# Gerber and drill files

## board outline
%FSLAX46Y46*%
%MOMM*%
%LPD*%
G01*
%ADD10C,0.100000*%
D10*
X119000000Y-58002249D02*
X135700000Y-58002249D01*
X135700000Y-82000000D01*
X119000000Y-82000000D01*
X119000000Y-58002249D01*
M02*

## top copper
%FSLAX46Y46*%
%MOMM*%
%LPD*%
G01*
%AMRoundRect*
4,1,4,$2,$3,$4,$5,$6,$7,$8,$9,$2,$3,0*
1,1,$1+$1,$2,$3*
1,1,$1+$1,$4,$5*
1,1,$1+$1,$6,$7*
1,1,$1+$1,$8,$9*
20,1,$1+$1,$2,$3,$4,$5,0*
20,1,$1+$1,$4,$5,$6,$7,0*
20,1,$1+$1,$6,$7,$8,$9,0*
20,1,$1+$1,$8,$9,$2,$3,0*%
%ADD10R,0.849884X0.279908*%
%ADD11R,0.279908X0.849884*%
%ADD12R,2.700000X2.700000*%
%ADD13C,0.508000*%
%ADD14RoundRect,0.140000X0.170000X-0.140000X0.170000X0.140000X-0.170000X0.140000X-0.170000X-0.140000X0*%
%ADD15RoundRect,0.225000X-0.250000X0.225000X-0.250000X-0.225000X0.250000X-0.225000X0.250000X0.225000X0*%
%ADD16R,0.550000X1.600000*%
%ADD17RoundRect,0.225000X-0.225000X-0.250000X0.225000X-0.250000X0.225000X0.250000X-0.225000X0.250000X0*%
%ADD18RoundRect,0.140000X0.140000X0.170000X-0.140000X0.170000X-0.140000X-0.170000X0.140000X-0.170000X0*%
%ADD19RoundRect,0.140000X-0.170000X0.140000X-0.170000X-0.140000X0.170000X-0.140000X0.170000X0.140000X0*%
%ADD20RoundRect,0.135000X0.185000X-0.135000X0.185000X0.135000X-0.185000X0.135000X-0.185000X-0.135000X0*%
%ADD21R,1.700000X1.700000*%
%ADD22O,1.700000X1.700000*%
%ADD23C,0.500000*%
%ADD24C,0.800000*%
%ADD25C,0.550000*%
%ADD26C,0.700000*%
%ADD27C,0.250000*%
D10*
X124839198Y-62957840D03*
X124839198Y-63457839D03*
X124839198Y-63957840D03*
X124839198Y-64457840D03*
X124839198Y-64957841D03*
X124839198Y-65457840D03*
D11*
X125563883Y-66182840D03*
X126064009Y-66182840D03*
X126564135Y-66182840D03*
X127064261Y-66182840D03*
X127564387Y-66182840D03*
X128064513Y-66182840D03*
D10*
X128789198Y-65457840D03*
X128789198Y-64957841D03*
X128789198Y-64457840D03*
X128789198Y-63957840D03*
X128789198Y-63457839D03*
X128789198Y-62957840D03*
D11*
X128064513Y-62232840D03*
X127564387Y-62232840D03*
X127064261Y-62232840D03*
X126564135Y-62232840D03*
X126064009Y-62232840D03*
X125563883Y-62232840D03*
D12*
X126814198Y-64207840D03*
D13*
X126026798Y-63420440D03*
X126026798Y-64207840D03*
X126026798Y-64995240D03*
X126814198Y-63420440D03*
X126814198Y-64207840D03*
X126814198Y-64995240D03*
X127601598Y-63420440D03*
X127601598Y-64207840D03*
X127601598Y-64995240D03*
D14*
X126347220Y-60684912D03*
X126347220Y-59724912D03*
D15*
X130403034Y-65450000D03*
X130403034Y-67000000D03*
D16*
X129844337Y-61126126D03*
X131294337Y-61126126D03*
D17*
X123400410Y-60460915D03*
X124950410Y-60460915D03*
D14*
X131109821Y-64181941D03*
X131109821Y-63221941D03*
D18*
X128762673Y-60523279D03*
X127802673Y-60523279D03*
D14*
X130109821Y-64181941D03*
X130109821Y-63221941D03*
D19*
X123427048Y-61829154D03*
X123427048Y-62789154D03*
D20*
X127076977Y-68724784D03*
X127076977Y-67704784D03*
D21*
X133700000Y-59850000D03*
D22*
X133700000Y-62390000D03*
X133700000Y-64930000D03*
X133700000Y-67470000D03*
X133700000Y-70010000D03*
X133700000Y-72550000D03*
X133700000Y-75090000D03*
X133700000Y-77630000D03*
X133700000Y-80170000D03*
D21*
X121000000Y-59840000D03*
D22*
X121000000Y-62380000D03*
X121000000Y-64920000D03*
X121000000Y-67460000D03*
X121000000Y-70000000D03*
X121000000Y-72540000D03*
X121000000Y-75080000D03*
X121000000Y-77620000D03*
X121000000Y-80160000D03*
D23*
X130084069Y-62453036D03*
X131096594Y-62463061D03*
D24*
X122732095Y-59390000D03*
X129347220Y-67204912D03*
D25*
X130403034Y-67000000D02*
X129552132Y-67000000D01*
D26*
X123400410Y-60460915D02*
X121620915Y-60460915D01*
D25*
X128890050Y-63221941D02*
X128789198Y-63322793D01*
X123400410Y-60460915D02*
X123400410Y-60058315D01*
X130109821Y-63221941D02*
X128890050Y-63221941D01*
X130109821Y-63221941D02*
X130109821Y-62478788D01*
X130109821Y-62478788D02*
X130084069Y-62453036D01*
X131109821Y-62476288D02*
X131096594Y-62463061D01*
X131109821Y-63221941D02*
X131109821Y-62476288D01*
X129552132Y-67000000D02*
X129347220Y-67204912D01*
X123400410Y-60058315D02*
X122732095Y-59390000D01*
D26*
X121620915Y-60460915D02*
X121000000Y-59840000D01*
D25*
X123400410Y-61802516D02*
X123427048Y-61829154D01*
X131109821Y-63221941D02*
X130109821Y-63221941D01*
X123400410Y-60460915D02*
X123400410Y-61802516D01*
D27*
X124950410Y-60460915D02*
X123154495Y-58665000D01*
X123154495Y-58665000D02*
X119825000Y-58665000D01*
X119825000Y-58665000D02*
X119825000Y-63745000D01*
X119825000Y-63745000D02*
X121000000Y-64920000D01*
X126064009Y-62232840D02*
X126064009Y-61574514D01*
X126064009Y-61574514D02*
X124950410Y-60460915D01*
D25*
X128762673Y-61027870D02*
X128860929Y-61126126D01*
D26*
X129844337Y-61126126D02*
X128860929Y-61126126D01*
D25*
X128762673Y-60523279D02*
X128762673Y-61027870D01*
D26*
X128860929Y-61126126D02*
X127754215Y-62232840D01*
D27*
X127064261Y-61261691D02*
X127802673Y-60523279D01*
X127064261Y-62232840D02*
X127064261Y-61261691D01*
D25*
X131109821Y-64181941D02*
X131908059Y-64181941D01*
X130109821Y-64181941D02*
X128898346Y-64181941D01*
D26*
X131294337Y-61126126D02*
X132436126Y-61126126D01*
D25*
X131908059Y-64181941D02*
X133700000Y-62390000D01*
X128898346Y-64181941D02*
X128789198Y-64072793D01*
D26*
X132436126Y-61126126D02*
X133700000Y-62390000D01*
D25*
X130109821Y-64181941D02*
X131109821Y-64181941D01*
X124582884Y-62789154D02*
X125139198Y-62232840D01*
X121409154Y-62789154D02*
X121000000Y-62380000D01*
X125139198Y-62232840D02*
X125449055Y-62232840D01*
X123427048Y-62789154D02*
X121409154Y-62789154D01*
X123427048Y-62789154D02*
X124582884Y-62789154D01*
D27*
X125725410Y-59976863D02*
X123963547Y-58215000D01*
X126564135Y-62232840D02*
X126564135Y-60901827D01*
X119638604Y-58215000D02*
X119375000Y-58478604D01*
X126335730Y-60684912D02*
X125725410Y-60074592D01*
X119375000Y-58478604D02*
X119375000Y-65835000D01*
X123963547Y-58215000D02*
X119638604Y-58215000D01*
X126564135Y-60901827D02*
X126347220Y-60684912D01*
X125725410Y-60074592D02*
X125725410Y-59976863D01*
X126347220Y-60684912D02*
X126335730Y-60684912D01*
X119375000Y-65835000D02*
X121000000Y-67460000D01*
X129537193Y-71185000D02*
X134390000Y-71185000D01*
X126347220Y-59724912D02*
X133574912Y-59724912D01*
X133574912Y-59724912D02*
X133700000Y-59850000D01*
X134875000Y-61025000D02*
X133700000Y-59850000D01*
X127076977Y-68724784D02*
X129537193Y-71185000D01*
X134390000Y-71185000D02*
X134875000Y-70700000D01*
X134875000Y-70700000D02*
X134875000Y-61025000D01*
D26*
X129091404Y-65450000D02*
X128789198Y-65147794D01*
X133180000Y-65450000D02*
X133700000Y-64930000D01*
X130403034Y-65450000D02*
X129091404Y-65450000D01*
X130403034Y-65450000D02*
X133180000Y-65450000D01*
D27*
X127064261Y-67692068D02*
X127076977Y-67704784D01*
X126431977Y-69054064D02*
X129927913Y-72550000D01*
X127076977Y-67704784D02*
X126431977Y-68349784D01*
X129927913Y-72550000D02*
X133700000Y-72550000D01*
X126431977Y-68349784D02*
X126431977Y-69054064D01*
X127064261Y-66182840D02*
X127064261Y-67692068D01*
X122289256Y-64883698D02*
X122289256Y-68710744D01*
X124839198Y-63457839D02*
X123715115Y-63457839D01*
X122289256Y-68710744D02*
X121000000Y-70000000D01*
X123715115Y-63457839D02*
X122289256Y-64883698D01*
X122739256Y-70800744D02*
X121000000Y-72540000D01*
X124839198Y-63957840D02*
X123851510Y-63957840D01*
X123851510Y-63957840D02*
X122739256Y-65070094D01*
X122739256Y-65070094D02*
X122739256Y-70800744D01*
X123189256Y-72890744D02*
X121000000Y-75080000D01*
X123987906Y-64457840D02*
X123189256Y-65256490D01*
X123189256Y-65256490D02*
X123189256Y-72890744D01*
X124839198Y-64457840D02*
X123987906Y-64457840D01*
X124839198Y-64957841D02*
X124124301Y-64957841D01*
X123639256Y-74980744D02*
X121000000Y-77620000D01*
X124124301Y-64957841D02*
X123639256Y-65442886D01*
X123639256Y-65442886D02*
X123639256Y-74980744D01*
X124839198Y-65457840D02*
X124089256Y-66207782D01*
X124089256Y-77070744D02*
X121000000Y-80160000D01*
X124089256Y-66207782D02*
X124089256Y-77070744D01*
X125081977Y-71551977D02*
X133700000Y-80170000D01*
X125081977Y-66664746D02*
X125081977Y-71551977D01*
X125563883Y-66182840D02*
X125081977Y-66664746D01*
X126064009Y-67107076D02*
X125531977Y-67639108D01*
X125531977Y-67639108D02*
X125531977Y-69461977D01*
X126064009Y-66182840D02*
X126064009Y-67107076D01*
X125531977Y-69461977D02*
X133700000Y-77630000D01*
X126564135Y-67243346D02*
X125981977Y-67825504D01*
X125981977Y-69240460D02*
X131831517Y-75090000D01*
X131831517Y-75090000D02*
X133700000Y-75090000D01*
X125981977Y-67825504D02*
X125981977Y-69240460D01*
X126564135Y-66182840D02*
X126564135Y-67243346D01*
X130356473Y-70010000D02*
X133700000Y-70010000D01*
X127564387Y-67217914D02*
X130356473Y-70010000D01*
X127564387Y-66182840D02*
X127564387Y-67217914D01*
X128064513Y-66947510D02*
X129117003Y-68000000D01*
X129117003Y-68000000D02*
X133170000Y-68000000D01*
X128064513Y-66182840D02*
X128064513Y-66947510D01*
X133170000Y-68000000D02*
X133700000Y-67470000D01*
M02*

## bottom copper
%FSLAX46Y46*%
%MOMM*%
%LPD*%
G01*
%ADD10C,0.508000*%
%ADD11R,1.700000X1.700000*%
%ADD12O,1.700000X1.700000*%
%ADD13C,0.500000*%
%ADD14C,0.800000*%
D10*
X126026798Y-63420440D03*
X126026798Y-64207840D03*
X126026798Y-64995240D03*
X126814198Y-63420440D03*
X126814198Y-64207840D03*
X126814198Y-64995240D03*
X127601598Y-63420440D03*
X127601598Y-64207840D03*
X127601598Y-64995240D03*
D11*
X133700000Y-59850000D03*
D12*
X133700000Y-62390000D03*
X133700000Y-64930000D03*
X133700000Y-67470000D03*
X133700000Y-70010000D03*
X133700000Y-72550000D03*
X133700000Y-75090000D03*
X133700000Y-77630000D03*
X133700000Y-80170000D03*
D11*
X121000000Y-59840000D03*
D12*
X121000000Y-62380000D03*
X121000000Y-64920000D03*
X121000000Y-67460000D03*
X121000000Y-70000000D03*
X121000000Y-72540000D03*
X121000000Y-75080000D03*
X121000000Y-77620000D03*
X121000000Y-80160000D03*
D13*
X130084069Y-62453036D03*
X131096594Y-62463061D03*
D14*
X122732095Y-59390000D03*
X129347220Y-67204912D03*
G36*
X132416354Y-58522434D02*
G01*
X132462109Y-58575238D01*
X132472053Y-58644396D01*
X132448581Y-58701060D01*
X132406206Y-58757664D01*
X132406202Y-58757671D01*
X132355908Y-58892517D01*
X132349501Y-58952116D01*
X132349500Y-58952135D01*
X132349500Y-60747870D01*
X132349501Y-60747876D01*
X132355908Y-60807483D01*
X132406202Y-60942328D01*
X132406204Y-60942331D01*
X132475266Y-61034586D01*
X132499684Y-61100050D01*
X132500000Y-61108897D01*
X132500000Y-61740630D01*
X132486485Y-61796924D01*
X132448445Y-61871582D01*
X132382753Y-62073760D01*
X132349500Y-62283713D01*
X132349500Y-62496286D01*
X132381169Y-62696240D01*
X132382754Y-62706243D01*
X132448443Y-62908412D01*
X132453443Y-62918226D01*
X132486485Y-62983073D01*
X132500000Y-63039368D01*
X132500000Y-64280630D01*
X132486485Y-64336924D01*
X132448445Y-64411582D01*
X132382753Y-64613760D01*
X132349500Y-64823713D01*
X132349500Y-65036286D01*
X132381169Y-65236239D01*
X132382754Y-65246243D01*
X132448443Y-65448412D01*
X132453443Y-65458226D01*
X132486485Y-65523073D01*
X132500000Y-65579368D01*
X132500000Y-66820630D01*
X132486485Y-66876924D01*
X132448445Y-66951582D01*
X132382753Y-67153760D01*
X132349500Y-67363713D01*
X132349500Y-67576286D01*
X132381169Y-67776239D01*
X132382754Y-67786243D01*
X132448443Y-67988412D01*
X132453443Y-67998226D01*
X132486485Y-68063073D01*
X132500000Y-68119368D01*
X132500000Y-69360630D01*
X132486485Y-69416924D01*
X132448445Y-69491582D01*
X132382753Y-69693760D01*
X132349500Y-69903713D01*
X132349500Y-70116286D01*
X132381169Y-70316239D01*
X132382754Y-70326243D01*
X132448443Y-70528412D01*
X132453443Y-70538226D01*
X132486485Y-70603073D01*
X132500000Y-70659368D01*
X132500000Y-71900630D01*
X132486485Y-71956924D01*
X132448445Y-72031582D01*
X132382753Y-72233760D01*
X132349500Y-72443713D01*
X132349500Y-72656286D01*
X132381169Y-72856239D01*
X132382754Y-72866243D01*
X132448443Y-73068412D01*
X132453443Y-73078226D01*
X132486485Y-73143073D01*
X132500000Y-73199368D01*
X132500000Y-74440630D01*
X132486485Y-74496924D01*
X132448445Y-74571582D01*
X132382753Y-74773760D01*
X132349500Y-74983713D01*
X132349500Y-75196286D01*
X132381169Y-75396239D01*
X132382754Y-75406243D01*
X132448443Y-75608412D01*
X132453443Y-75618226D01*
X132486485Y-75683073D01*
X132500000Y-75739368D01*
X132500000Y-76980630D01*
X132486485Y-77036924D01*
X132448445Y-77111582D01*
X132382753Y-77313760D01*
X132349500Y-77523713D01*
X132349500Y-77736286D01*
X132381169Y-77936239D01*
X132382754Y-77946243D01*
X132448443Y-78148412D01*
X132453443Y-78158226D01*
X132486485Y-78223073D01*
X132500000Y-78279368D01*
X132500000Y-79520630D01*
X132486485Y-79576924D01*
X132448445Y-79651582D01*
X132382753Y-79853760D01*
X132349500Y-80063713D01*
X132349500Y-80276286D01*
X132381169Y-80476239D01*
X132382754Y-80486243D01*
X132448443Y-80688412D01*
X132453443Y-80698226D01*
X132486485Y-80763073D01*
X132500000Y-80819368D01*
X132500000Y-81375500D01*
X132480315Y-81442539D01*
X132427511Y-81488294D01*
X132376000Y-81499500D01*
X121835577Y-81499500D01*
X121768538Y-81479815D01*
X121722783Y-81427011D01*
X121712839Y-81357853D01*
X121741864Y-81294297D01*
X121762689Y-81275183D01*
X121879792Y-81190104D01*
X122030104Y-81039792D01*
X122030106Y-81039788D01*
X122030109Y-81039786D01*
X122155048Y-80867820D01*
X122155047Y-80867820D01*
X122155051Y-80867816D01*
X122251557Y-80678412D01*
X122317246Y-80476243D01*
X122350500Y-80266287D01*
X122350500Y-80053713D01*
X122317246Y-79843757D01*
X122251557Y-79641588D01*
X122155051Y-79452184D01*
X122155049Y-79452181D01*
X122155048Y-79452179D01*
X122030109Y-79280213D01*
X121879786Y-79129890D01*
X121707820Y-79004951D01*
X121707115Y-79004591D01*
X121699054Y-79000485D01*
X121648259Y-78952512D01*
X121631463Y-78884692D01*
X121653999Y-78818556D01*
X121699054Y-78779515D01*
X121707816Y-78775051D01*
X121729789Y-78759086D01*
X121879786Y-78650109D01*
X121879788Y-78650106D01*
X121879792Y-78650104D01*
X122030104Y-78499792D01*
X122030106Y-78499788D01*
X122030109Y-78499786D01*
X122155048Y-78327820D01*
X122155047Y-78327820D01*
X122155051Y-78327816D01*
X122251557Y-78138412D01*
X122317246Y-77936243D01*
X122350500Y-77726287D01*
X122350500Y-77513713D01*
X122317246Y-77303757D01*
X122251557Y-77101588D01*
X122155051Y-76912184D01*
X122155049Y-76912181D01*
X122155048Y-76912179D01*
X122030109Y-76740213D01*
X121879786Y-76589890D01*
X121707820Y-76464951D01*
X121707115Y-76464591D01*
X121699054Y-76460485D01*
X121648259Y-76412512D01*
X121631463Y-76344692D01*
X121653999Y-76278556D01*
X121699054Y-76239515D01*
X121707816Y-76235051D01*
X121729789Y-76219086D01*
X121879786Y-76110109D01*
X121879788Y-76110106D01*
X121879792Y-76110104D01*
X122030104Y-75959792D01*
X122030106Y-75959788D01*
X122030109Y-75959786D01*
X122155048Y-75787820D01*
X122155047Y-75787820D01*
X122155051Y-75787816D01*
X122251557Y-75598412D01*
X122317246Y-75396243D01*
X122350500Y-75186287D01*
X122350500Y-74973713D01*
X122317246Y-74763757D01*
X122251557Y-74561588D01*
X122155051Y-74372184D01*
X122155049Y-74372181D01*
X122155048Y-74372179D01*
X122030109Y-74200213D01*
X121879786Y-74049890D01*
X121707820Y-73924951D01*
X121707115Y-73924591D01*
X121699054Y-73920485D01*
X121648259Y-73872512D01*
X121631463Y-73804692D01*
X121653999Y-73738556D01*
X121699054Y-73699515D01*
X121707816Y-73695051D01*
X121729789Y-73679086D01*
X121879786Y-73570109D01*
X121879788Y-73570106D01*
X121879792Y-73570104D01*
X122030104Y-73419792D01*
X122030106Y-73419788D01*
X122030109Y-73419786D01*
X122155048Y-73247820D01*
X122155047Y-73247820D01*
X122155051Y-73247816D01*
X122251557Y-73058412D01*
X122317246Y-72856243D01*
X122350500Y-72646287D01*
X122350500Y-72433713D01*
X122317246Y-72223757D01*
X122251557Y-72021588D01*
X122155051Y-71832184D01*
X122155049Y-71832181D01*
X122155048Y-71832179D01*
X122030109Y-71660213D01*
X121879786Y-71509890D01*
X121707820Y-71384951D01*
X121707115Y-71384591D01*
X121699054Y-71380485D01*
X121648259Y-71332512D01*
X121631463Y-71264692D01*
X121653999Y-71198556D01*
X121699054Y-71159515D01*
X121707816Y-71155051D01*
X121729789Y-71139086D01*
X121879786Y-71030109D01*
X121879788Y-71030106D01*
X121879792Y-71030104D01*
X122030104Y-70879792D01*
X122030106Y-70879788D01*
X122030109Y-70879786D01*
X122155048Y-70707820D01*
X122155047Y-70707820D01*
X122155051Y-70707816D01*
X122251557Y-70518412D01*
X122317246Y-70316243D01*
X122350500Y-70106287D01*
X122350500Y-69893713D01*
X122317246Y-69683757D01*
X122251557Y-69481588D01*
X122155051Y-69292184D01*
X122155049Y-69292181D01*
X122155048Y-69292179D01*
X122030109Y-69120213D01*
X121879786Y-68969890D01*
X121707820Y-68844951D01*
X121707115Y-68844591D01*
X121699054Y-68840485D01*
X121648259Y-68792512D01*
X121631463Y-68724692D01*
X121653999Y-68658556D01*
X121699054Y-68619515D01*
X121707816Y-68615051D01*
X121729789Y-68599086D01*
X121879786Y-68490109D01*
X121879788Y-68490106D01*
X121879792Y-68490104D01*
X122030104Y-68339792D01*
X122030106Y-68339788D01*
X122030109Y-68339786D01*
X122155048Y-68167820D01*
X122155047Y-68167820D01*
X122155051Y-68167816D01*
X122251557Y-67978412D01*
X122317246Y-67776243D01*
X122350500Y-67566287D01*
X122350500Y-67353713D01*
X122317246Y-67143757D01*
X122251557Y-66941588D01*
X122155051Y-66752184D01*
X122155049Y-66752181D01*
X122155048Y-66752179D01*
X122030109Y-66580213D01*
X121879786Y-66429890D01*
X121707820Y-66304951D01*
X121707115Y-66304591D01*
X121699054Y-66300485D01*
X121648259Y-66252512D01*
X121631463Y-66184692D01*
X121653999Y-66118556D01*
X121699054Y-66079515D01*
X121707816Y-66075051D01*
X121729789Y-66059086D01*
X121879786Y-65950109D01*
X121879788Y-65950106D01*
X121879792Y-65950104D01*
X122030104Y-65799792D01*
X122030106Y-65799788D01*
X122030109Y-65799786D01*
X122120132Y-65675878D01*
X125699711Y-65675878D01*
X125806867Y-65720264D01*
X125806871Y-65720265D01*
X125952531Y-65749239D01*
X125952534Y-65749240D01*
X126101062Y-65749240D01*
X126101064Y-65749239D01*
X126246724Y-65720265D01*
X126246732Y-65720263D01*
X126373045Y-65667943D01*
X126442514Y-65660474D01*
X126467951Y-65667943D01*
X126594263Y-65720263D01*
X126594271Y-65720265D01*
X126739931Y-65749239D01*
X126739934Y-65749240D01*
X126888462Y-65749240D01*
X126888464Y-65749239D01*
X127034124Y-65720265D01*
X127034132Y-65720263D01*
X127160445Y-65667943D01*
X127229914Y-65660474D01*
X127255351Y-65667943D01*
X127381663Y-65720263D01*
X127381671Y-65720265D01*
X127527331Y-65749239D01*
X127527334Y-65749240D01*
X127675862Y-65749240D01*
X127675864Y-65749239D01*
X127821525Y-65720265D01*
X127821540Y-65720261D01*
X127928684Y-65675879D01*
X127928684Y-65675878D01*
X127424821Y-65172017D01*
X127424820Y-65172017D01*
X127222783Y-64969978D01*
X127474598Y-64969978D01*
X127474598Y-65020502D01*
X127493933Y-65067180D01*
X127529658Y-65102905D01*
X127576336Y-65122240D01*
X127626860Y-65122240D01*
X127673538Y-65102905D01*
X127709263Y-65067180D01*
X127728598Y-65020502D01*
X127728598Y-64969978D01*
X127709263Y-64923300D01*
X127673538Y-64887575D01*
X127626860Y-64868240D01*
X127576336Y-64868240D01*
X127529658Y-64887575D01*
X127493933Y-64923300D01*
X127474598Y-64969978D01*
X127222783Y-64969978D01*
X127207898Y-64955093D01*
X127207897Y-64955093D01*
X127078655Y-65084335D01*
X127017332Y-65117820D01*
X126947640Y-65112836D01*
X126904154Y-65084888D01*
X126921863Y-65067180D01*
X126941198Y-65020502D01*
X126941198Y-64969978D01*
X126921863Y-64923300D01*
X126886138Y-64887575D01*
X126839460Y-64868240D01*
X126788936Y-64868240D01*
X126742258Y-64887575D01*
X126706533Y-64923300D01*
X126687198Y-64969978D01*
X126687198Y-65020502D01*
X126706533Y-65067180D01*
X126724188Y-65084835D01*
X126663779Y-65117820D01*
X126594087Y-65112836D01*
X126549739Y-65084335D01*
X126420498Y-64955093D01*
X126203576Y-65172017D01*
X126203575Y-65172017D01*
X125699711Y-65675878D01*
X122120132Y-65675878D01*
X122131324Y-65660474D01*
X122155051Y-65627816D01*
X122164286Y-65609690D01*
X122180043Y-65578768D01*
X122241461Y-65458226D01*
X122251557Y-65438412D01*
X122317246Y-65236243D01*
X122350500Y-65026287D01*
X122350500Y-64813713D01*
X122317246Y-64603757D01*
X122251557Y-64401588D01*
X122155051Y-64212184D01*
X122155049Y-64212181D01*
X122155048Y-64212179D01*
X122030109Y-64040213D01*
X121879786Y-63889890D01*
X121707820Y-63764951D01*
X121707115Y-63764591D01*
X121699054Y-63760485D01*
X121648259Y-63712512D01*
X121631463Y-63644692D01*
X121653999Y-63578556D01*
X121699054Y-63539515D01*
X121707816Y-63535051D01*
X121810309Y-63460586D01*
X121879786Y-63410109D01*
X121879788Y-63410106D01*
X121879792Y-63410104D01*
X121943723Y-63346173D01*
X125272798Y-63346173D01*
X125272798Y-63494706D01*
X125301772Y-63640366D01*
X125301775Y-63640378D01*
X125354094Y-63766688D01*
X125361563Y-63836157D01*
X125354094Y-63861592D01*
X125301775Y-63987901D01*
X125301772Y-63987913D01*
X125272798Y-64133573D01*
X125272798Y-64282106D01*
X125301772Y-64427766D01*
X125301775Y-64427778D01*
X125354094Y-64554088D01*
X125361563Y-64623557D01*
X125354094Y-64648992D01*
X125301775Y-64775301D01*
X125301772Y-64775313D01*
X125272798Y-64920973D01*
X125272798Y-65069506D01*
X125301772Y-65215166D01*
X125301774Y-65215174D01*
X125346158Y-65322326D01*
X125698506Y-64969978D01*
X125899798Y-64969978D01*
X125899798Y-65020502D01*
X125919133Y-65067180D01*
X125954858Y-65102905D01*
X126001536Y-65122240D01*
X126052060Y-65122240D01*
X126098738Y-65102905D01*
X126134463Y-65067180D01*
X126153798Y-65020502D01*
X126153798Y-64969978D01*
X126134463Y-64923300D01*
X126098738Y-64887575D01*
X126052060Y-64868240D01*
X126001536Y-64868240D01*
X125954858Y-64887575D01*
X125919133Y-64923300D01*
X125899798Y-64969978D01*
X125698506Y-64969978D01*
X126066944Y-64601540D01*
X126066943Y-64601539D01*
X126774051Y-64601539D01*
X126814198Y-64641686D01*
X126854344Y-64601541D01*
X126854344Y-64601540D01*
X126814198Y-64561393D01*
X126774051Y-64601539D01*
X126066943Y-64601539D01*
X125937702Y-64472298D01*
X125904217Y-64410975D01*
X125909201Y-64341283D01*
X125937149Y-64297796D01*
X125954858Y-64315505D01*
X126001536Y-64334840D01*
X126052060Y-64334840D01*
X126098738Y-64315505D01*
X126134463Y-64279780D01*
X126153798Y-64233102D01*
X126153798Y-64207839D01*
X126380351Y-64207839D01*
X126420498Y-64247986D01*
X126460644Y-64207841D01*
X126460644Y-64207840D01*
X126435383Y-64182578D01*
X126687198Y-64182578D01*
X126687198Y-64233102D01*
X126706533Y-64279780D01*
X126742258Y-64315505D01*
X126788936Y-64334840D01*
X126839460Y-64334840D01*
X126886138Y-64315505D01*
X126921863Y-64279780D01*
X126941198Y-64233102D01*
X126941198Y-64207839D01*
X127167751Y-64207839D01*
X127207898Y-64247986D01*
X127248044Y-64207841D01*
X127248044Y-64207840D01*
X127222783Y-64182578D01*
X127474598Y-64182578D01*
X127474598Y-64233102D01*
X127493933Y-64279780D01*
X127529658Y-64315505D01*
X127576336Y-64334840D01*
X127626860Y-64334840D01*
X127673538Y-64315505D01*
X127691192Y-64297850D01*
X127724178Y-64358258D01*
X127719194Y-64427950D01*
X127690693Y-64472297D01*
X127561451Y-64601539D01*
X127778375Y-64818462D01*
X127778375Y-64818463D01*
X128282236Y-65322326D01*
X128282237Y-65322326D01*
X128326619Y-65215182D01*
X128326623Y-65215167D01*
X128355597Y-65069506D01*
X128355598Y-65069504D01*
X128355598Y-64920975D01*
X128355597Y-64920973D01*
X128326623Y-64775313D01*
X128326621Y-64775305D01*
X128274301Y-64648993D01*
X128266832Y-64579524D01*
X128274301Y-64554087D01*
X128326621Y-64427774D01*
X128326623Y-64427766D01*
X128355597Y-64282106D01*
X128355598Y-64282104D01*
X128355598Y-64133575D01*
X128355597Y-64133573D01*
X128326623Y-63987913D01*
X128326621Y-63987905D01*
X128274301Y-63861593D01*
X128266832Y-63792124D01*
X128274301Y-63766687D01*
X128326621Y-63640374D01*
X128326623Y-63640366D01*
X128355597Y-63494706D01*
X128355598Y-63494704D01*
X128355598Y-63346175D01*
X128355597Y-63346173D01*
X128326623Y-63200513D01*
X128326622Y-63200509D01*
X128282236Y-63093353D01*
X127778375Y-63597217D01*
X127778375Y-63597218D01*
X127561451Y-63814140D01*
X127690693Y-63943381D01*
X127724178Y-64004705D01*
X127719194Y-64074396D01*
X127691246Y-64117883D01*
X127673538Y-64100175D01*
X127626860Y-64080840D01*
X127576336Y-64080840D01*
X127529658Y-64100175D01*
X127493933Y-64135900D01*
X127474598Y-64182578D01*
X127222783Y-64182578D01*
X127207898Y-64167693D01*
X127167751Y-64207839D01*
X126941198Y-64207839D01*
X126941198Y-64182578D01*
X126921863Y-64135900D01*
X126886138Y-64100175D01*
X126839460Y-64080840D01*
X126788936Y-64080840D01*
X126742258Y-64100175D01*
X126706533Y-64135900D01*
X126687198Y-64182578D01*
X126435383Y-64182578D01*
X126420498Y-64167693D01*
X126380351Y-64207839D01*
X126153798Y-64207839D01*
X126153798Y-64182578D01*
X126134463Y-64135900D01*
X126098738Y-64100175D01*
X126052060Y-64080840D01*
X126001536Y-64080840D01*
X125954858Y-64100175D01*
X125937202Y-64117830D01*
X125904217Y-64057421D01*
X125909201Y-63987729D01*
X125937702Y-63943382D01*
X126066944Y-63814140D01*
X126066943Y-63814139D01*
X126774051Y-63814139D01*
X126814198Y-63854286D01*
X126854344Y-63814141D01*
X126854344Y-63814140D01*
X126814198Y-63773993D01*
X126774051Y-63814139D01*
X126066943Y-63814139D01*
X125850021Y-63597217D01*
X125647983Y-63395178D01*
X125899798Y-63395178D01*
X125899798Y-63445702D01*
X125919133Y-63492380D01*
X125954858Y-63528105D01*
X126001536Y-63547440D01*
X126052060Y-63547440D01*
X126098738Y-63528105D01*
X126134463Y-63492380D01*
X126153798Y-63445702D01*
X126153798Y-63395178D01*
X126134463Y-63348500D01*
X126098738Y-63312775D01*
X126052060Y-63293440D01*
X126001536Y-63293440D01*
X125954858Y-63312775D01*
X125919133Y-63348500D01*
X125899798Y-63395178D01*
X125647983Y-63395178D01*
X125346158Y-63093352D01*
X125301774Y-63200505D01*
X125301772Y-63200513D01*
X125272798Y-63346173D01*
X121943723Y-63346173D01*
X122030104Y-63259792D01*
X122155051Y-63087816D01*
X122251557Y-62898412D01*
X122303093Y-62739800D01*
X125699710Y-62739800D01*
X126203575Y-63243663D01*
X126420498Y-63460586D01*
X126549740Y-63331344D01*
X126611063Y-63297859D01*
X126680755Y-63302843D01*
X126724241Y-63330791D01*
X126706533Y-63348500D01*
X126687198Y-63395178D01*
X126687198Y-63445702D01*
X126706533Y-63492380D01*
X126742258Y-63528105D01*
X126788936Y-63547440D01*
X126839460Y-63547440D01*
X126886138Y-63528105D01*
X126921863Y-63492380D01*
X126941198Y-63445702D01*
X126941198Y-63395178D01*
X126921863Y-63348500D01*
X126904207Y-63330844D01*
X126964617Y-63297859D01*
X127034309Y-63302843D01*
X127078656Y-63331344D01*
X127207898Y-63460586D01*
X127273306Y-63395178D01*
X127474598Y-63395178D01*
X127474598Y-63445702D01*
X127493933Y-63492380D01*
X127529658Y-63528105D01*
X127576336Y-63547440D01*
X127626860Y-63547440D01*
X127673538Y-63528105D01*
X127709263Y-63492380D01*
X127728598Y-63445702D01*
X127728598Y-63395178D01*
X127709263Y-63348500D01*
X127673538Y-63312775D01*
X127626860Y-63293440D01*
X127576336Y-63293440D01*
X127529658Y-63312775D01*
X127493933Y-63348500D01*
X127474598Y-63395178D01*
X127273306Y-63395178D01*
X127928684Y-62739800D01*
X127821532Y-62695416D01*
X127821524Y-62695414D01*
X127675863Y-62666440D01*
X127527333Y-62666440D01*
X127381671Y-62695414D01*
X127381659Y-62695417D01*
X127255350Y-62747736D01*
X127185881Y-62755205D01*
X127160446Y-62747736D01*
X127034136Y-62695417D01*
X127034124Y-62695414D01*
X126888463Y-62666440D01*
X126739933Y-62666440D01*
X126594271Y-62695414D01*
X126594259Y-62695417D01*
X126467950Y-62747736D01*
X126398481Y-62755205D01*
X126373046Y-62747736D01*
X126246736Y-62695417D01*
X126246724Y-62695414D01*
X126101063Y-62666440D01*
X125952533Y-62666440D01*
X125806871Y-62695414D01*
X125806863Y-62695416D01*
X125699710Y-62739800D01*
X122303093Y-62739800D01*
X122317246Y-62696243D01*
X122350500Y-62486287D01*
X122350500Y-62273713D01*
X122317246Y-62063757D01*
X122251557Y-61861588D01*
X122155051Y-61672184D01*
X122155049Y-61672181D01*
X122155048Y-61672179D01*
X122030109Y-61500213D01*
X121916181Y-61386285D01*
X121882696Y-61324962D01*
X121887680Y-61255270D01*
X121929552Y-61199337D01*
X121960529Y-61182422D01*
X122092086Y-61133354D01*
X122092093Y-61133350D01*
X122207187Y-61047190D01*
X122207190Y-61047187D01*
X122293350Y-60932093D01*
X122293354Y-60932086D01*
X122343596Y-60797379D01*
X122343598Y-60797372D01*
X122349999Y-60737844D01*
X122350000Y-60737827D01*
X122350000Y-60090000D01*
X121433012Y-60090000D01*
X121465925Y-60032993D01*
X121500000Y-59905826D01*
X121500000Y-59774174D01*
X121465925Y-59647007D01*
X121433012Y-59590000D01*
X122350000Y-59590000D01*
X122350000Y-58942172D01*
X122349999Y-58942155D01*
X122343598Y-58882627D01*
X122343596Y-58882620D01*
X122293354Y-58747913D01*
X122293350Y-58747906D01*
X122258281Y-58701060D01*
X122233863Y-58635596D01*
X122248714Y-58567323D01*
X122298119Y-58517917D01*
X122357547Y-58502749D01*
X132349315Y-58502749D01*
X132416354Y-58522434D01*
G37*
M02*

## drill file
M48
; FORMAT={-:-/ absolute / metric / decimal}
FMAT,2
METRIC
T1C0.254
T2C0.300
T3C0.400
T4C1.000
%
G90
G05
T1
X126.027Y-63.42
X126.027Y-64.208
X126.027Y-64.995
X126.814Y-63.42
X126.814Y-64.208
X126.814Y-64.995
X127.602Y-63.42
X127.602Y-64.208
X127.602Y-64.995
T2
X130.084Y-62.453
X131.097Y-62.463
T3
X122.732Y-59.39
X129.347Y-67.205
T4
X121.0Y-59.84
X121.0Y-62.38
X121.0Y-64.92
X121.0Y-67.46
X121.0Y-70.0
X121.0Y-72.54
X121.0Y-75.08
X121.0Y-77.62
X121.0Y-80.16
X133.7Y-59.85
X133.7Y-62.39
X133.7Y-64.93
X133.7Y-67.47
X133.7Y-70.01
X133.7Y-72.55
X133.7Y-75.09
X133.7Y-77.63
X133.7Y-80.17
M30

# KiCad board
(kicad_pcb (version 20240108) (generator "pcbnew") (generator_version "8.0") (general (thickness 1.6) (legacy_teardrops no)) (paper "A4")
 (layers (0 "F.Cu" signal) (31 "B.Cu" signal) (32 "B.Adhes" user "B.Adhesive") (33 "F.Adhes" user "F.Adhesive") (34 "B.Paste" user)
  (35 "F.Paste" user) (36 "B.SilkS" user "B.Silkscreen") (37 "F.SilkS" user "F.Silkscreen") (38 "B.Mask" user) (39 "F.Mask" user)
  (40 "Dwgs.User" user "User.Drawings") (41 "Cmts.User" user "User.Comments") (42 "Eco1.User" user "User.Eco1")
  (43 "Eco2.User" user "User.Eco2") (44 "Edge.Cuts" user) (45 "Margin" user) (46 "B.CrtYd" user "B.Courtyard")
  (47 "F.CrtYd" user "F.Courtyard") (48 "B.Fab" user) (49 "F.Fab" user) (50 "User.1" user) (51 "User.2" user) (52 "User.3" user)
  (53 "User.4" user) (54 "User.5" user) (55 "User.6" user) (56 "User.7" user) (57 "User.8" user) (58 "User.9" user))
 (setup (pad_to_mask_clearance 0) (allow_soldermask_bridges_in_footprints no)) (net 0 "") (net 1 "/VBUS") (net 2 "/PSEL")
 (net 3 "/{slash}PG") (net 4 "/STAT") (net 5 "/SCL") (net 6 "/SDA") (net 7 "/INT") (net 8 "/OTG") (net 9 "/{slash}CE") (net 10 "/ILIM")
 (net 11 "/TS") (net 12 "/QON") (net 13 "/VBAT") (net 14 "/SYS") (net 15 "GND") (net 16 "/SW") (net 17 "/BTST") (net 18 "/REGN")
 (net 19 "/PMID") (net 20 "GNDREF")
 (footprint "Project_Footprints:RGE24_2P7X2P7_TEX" (layer "F.Cu") (at 126.814198 64.20784)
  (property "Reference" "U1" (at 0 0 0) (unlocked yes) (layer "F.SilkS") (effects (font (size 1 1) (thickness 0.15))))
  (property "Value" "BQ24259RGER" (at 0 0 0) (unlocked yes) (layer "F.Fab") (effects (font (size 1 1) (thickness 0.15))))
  (pad "1" smd rect (at -1.975 -1.25 90) (size 0.279908 0.849884) (layers "F.Cu" "F.Mask") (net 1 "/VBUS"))
  (pad "2" smd rect (at -1.975 -0.750001 90) (size 0.279908 0.849884) (layers "F.Cu" "F.Mask") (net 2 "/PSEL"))
  (pad "3" smd rect (at -1.975 -0.25 90) (size 0.279908 0.849884) (layers "F.Cu" "F.Mask") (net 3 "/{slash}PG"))
  (pad "4" smd rect (at -1.975 0.25 90) (size 0.279908 0.849884) (layers "F.Cu" "F.Mask") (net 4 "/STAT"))
  (pad "5" smd rect (at -1.975 0.750001 90) (size 0.279908 0.849884) (layers "F.Cu" "F.Mask") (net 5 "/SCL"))
  (pad "6" smd rect (at -1.975 1.25 90) (size 0.279908 0.849884) (layers "F.Cu" "F.Mask") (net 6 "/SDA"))
  (pad "7" smd rect (at -1.250315 1.975) (size 0.279908 0.849884) (layers "F.Cu" "F.Mask") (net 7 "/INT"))
  (pad "8" smd rect (at -0.750189 1.975) (size 0.279908 0.849884) (layers "F.Cu" "F.Mask") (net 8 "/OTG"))
  (pad "9" smd rect (at -0.250063 1.975) (size 0.279908 0.849884) (layers "F.Cu" "F.Mask") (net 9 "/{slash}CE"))
  (pad "10" smd rect (at 0.250063 1.975) (size 0.279908 0.849884) (layers "F.Cu" "F.Mask") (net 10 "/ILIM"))
  (pad "11" smd rect (at 0.750189 1.975) (size 0.279908 0.849884) (layers "F.Cu" "F.Mask") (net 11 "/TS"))
  (pad "12" smd rect (at 1.250315 1.975) (size 0.279908 0.849884) (layers "F.Cu" "F.Mask") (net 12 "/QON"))
  (pad "13" smd rect (at 1.975 1.25 90) (size 0.279908 0.849884) (layers "F.Cu" "F.Mask") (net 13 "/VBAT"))
  (pad "14" smd rect (at 1.975 0.750001 90) (size 0.279908 0.849884) (layers "F.Cu" "F.Mask") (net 13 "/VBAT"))
  (pad "15" smd rect (at 1.975 0.25 90) (size 0.279908 0.849884) (layers "F.Cu" "F.Mask") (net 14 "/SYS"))
  (pad "16" smd rect (at 1.975 -0.25 90) (size 0.279908 0.849884) (layers "F.Cu" "F.Mask") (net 14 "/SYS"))
  (pad "17" smd rect (at 1.975 -0.750001 90) (size 0.279908 0.849884) (layers "F.Cu" "F.Mask") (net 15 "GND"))
  (pad "18" smd rect (at 1.975 -1.25 90) (size 0.279908 0.849884) (layers "F.Cu" "F.Mask") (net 15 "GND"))
  (pad "19" smd rect (at 1.250315 -1.975) (size 0.279908 0.849884) (layers "F.Cu" "F.Mask") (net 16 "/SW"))
  (pad "20" smd rect (at 0.750189 -1.975) (size 0.279908 0.849884) (layers "F.Cu" "F.Mask") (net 16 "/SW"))
  (pad "21" smd rect (at 0.250063 -1.975) (size 0.279908 0.849884) (layers "F.Cu" "F.Mask") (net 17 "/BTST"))
  (pad "22" smd rect (at -0.250063 -1.975) (size 0.279908 0.849884) (layers "F.Cu" "F.Mask") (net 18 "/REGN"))
  (pad "23" smd rect (at -0.750189 -1.975) (size 0.279908 0.849884) (layers "F.Cu" "F.Mask") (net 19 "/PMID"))
  (pad "24" smd rect (at -1.250315 -1.975) (size 0.279908 0.849884) (layers "F.Cu" "F.Mask") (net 1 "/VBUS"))
  (pad "25" smd rect (at 0 0) (size 2.7 2.7) (layers "F.Cu") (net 15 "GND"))
  (pad "V" thru_hole circle (at -0.7874 -0.7874) (size 0.508 0.508) (drill 0.254) (layers "*.Cu" "*.Mask") (remove_unused_layers no)
   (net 15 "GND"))
  (pad "V" thru_hole circle (at -0.7874 0) (size 0.508 0.508) (drill 0.254) (layers "*.Cu" "*.Mask") (remove_unused_layers no)
   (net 15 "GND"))
  (pad "V" thru_hole circle (at -0.7874 0.7874) (size 0.508 0.508) (drill 0.254) (layers "*.Cu" "*.Mask") (remove_unused_layers no)
   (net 15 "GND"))
  (pad "V" thru_hole circle (at 0 -0.7874) (size 0.508 0.508) (drill 0.254) (layers "*.Cu" "*.Mask") (remove_unused_layers no)
   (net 15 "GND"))
  (pad "V" thru_hole circle (at 0 0) (size 0.508 0.508) (drill 0.254) (layers "*.Cu" "*.Mask") (remove_unused_layers no) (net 15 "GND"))
  (pad "V" thru_hole circle (at 0 0.7874) (size 0.508 0.508) (drill 0.254) (layers "*.Cu" "*.Mask") (remove_unused_layers no) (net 15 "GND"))
  (pad "V" thru_hole circle (at 0.7874 -0.7874) (size 0.508 0.508) (drill 0.254) (layers "*.Cu" "*.Mask") (remove_unused_layers no)
   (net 15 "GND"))
  (pad "V" thru_hole circle (at 0.7874 0) (size 0.508 0.508) (drill 0.254) (layers "*.Cu" "*.Mask") (remove_unused_layers no) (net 15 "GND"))
  (pad "V" thru_hole circle (at 0.7874 0.7874) (size 0.508 0.508) (drill 0.254) (layers "*.Cu" "*.Mask") (remove_unused_layers no)
   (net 15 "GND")))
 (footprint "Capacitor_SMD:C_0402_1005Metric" (layer "F.Cu") (at 126.34722 60.204912 90)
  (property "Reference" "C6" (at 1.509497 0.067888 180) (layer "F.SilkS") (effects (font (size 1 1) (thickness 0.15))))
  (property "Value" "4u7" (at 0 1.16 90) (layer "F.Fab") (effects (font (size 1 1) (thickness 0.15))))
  (pad "1" smd roundrect (at -0.48 0 90) (size 0.56 0.62) (layers "F.Cu" "F.Paste" "F.Mask") (roundrect_rratio 0.25) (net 18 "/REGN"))
  (pad "2" smd roundrect (at 0.48 0 90) (size 0.56 0.62) (layers "F.Cu" "F.Paste" "F.Mask") (roundrect_rratio 0.25) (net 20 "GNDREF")))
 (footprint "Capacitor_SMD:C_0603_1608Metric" (layer "F.Cu") (at 130.403034 66.225 -90)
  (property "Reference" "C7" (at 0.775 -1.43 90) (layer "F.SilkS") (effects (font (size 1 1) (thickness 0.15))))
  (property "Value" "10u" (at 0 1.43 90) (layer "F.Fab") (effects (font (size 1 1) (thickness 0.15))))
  (pad "1" smd roundrect (at -0.775 0 270) (size 0.9 0.95) (layers "F.Cu" "F.Paste" "F.Mask") (roundrect_rratio 0.25) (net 13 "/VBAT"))
  (pad "2" smd roundrect (at 0.775 0 270) (size 0.9 0.95) (layers "F.Cu" "F.Paste" "F.Mask") (roundrect_rratio 0.25) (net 15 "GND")))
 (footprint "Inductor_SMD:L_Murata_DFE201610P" (layer "F.Cu") (at 130.569337 61.126126)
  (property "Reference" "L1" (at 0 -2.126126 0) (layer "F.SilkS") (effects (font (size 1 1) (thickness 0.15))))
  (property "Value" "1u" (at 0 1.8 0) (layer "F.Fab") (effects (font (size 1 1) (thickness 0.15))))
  (pad "1" smd rect (at -0.725 0) (size 0.55 1.6) (layers "F.Cu" "F.Paste" "F.Mask") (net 16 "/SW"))
  (pad "2" smd rect (at 0.725 0) (size 0.55 1.6) (layers "F.Cu" "F.Paste" "F.Mask") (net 14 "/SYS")))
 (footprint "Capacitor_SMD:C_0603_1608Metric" (layer "F.Cu") (at 124.17541 60.460915)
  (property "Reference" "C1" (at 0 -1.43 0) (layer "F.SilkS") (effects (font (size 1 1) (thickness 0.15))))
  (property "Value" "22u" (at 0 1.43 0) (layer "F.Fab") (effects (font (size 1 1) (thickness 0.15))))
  (pad "1" smd roundrect (at -0.775 0) (size 0.9 0.95) (layers "F.Cu" "F.Paste" "F.Mask") (roundrect_rratio 0.25) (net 15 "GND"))
  (pad "2" smd roundrect (at 0.775 0) (size 0.9 0.95) (layers "F.Cu" "F.Paste" "F.Mask") (roundrect_rratio 0.25) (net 19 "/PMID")))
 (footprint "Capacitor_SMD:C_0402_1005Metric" (layer "F.Cu") (at 131.109821 63.701941 90)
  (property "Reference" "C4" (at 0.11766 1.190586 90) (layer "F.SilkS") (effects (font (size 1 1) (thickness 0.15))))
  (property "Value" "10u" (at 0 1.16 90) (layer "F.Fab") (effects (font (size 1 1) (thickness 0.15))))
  (pad "1" smd roundrect (at -0.48 0 90) (size 0.56 0.62) (layers "F.Cu" "F.Paste" "F.Mask") (roundrect_rratio 0.25) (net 14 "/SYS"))
  (pad "2" smd roundrect (at 0.48 0 90) (size 0.56 0.62) (layers "F.Cu" "F.Paste" "F.Mask") (roundrect_rratio 0.25) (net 15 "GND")))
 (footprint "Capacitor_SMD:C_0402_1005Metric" (layer "F.Cu") (at 128.282673 60.523279 180)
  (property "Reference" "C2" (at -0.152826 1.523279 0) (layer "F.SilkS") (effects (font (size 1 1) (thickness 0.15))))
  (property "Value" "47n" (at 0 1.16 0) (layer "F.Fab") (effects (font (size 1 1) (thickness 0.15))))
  (pad "1" smd roundrect (at -0.48 0 180) (size 0.56 0.62) (layers "F.Cu" "F.Paste" "F.Mask") (roundrect_rratio 0.25) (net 16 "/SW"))
  (pad "2" smd roundrect (at 0.48 0 180) (size 0.56 0.62) (layers "F.Cu" "F.Paste" "F.Mask") (roundrect_rratio 0.25) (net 17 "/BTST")))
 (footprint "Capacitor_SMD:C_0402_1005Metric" (layer "F.Cu") (at 130.109821 63.701941 90)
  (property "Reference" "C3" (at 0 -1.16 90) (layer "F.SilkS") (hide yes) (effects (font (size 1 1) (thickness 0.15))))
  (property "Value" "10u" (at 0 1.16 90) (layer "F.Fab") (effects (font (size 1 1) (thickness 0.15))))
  (pad "1" smd roundrect (at -0.48 0 90) (size 0.56 0.62) (layers "F.Cu" "F.Paste" "F.Mask") (roundrect_rratio 0.25) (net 14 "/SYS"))
  (pad "2" smd roundrect (at 0.48 0 90) (size 0.56 0.62) (layers "F.Cu" "F.Paste" "F.Mask") (roundrect_rratio 0.25) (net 15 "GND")))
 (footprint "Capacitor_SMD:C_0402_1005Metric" (layer "F.Cu") (at 123.427048 62.309154 -90)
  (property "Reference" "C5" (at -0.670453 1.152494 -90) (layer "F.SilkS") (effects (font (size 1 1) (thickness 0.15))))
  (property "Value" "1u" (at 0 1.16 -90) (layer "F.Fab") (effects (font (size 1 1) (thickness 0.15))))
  (pad "1" smd roundrect (at -0.48 0 270) (size 0.56 0.62) (layers "F.Cu" "F.Paste" "F.Mask") (roundrect_rratio 0.25) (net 15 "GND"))
  (pad "2" smd roundrect (at 0.48 0 270) (size 0.56 0.62) (layers "F.Cu" "F.Paste" "F.Mask") (roundrect_rratio 0.25) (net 1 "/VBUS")))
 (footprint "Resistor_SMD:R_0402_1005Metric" (layer "F.Cu") (at 127.076977 68.214784 90)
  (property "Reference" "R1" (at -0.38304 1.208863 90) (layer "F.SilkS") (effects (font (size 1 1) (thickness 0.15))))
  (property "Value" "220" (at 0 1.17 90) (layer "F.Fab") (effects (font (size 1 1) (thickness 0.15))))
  (pad "1" smd roundrect (at -0.51 0 90) (size 0.54 0.64) (layers "F.Cu" "F.Paste" "F.Mask") (roundrect_rratio 0.25) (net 20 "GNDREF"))
  (pad "2" smd roundrect (at 0.51 0 90) (size 0.54 0.64) (layers "F.Cu" "F.Paste" "F.Mask") (roundrect_rratio 0.25) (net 10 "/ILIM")))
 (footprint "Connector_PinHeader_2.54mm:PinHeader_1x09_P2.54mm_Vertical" (layer "B.Cu") (at 133.7 59.85 180)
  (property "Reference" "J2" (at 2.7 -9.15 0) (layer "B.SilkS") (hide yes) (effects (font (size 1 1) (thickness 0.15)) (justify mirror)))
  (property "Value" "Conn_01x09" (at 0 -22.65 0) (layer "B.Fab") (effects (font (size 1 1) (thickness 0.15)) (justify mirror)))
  (pad "1" thru_hole rect (at 0 0 180) (size 1.7 1.7) (drill 1) (layers "*.Cu" "*.Mask") (remove_unused_layers no) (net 20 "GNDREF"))
  (pad "2" thru_hole oval (at 0 -2.54 180) (size 1.7 1.7) (drill 1) (layers "*.Cu" "*.Mask") (remove_unused_layers no) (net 14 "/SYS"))
  (pad "3" thru_hole oval (at 0 -5.08 180) (size 1.7 1.7) (drill 1) (layers "*.Cu" "*.Mask") (remove_unused_layers no) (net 13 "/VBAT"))
  (pad "4" thru_hole oval (at 0 -7.62 180) (size 1.7 1.7) (drill 1) (layers "*.Cu" "*.Mask") (remove_unused_layers no) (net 12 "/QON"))
  (pad "5" thru_hole oval (at 0 -10.16 180) (size 1.7 1.7) (drill 1) (layers "*.Cu" "*.Mask") (remove_unused_layers no) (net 11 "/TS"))
  (pad "6" thru_hole oval (at 0 -12.7 180) (size 1.7 1.7) (drill 1) (layers "*.Cu" "*.Mask") (remove_unused_layers no) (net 10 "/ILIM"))
  (pad "7" thru_hole oval (at 0 -15.24 180) (size 1.7 1.7) (drill 1) (layers "*.Cu" "*.Mask") (remove_unused_layers no) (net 9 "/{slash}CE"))
  (pad "8" thru_hole oval (at 0 -17.78 180) (size 1.7 1.7) (drill 1) (layers "*.Cu" "*.Mask") (remove_unused_layers no) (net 8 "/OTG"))
  (pad "9" thru_hole oval (at 0 -20.32 180) (size 1.7 1.7) (drill 1) (layers "*.Cu" "*.Mask") (remove_unused_layers no) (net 7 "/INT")))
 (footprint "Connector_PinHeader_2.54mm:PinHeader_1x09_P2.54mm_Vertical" (layer "B.Cu") (at 121 59.84 180)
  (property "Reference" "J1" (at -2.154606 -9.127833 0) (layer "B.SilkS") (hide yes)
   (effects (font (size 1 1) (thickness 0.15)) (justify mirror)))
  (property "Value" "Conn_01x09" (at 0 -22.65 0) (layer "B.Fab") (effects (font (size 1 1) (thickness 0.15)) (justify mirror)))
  (pad "1" thru_hole rect (at 0 0 180) (size 1.7 1.7) (drill 1) (layers "*.Cu" "*.Mask") (remove_unused_layers no) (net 15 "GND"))
  (pad "2" thru_hole oval (at 0 -2.54 180) (size 1.7 1.7) (drill 1) (layers "*.Cu" "*.Mask") (remove_unused_layers no) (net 1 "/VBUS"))
  (pad "3" thru_hole oval (at 0 -5.08 180) (size 1.7 1.7) (drill 1) (layers "*.Cu" "*.Mask") (remove_unused_layers no) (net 19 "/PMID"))
  (pad "4" thru_hole oval (at 0 -7.62 180) (size 1.7 1.7) (drill 1) (layers "*.Cu" "*.Mask") (remove_unused_layers no) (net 18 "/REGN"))
  (pad "5" thru_hole oval (at 0 -10.16 180) (size 1.7 1.7) (drill 1) (layers "*.Cu" "*.Mask") (remove_unused_layers no) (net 2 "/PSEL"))
  (pad "6" thru_hole oval (at 0 -12.7 180) (size 1.7 1.7) (drill 1) (layers "*.Cu" "*.Mask") (remove_unused_layers no) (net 3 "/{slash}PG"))
  (pad "7" thru_hole oval (at 0 -15.24 180) (size 1.7 1.7) (drill 1) (layers "*.Cu" "*.Mask") (remove_unused_layers no) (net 4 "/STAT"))
  (pad "8" thru_hole oval (at 0 -17.78 180) (size 1.7 1.7) (drill 1) (layers "*.Cu" "*.Mask") (remove_unused_layers no) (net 5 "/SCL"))
  (pad "9" thru_hole oval (at 0 -20.32 180) (size 1.7 1.7) (drill 1) (layers "*.Cu" "*.Mask") (remove_unused_layers no) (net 6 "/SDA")))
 (gr_rect (start 119 58.002249) (end 135.7 82) (stroke (width 0.1) (type default)) (fill none) (layer "Edge.Cuts"))
 (segment (start 130.403034 67) (end 129.552132 67) (width 0.55) (layer "F.Cu") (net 15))
 (segment (start 123.40041 60.460915) (end 121.620915 60.460915) (width 0.7) (layer "F.Cu") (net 15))
 (segment (start 128.89005 63.221941) (end 128.789198 63.322793) (width 0.55) (layer "F.Cu") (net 15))
 (segment (start 123.40041 60.460915) (end 123.40041 60.058315) (width 0.55) (layer "F.Cu") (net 15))
 (segment (start 130.109821 63.221941) (end 128.89005 63.221941) (width 0.55) (layer "F.Cu") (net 15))
 (segment (start 130.109821 63.221941) (end 130.109821 62.478788) (width 0.55) (layer "F.Cu") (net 15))
 (segment (start 130.109821 62.478788) (end 130.084069 62.453036) (width 0.55) (layer "F.Cu") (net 15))
 (segment (start 131.109821 62.476288) (end 131.096594 62.463061) (width 0.55) (layer "F.Cu") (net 15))
 (segment (start 131.109821 63.221941) (end 131.109821 62.476288) (width 0.55) (layer "F.Cu") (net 15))
 (segment (start 129.552132 67) (end 129.34722 67.204912) (width 0.55) (layer "F.Cu") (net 15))
 (segment (start 123.40041 60.058315) (end 122.732095 59.39) (width 0.55) (layer "F.Cu") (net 15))
 (segment (start 121.620915 60.460915) (end 121 59.84) (width 0.7) (layer "F.Cu") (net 15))
 (segment (start 123.40041 61.802516) (end 123.427048 61.829154) (width 0.55) (layer "F.Cu") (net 15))
 (segment (start 131.109821 63.221941) (end 130.109821 63.221941) (width 0.55) (layer "F.Cu") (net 15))
 (segment (start 123.40041 60.460915) (end 123.40041 61.802516) (width 0.55) (layer "F.Cu") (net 15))
 (via (at 130.084069 62.453036) (size 0.5) (drill 0.3) (layers "F.Cu" "B.Cu") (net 15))
 (via (at 131.096594 62.463061) (size 0.5) (drill 0.3) (layers "F.Cu" "B.Cu") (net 15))
 (via (at 122.732095 59.39) (size 0.8) (drill 0.4) (layers "F.Cu" "B.Cu") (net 15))
 (via (at 129.34722 67.204912) (size 0.8) (drill 0.4) (layers "F.Cu" "B.Cu") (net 15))
 (segment (start 124.95041 60.460915) (end 123.154495 58.665) (width 0.25) (layer "F.Cu") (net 19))
 (segment (start 123.154495 58.665) (end 119.825 58.665) (width 0.25) (layer "F.Cu") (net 19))
 (segment (start 119.825 58.665) (end 119.825 63.745) (width 0.25) (layer "F.Cu") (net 19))
 (segment (start 119.825 63.745) (end 121 64.92) (width 0.25) (layer "F.Cu") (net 19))
 (segment (start 126.064009 62.23284) (end 126.064009 61.574514) (width 0.25) (layer "F.Cu") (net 19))
 (segment (start 126.064009 61.574514) (end 124.95041 60.460915) (width 0.25) (layer "F.Cu") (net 19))
 (segment (start 128.762673 61.02787) (end 128.860929 61.126126) (width 0.55) (layer "F.Cu") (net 16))
 (segment (start 129.844337 61.126126) (end 128.860929 61.126126) (width 0.7) (layer "F.Cu") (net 16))
 (segment (start 128.762673 60.523279) (end 128.762673 61.02787) (width 0.55) (layer "F.Cu") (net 16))
 (segment (start 128.860929 61.126126) (end 127.754215 62.23284) (width 0.7) (layer "F.Cu") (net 16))
 (segment (start 127.064261 61.261691) (end 127.802673 60.523279) (width 0.25) (layer "F.Cu") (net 17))
 (segment (start 127.064261 62.23284) (end 127.064261 61.261691) (width 0.25) (layer "F.Cu") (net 17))
 (segment (start 131.109821 64.181941) (end 131.908059 64.181941) (width 0.55) (layer "F.Cu") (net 14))
 (segment (start 130.109821 64.181941) (end 128.898346 64.181941) (width 0.55) (layer "F.Cu") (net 14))
 (segment (start 131.294337 61.126126) (end 132.436126 61.126126) (width 0.7) (layer "F.Cu") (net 14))
 (segment (start 131.908059 64.181941) (end 133.7 62.39) (width 0.55) (layer "F.Cu") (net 14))
 (segment (start 128.898346 64.181941) (end 128.789198 64.072793) (width 0.55) (layer "F.Cu") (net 14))
 (segment (start 132.436126 61.126126) (end 133.7 62.39) (width 0.7) (layer "F.Cu") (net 14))
 (segment (start 130.109821 64.181941) (end 131.109821 64.181941) (width 0.55) (layer "F.Cu") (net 14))
 (segment (start 124.582884 62.789154) (end 125.139198 62.23284) (width 0.55) (layer "F.Cu") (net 1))
 (segment (start 121.409154 62.789154) (end 121 62.38) (width 0.55) (layer "F.Cu") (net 1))
 (segment (start 125.139198 62.23284) (end 125.449055 62.23284) (width 0.55) (layer "F.Cu") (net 1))
 (segment (start 123.427048 62.789154) (end 121.409154 62.789154) (width 0.55) (layer "F.Cu") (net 1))
 (segment (start 123.427048 62.789154) (end 124.582884 62.789154) (width 0.55) (layer "F.Cu") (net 1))
 (segment (start 125.72541 59.976863) (end 123.963547 58.215) (width 0.25) (layer "F.Cu") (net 18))
 (segment (start 126.564135 62.23284) (end 126.564135 60.901827) (width 0.25) (layer "F.Cu") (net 18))
 (segment (start 119.638604 58.215) (end 119.375 58.478604) (width 0.25) (layer "F.Cu") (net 18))
 (segment (start 126.33573 60.684912) (end 125.72541 60.074592) (width 0.25) (layer "F.Cu") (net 18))
 (segment (start 119.375 58.478604) (end 119.375 65.835) (width 0.25) (layer "F.Cu") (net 18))
 (segment (start 123.963547 58.215) (end 119.638604 58.215) (width 0.25) (layer "F.Cu") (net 18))
 (segment (start 126.564135 60.901827) (end 126.34722 60.684912) (width 0.25) (layer "F.Cu") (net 18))
 (segment (start 125.72541 60.074592) (end 125.72541 59.976863) (width 0.25) (layer "F.Cu") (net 18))
 (segment (start 126.34722 60.684912) (end 126.33573 60.684912) (width 0.25) (layer "F.Cu") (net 18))
 (segment (start 119.375 65.835) (end 121 67.46) (width 0.25) (layer "F.Cu") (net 18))
 (segment (start 129.537193 71.185) (end 134.39 71.185) (width 0.25) (layer "F.Cu") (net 20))
 (segment (start 126.34722 59.724912) (end 133.574912 59.724912) (width 0.25) (layer "F.Cu") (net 20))
 (segment (start 133.574912 59.724912) (end 133.7 59.85) (width 0.25) (layer "F.Cu") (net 20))
 (segment (start 134.875 61.025) (end 133.7 59.85) (width 0.25) (layer "F.Cu") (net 20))
 (segment (start 127.076977 68.724784) (end 129.537193 71.185) (width 0.25) (layer "F.Cu") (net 20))
 (segment (start 134.39 71.185) (end 134.875 70.7) (width 0.25) (layer "F.Cu") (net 20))
 (segment (start 134.875 70.7) (end 134.875 61.025) (width 0.25) (layer "F.Cu") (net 20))
 (segment (start 129.091404 65.45) (end 128.789198 65.147794) (width 0.7) (layer "F.Cu") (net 13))
 (segment (start 133.18 65.45) (end 133.7 64.93) (width 0.7) (layer "F.Cu") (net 13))
 (segment (start 130.403034 65.45) (end 129.091404 65.45) (width 0.7) (layer "F.Cu") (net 13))
 (segment (start 130.403034 65.45) (end 133.18 65.45) (width 0.7) (layer "F.Cu") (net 13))
 (segment (start 127.064261 67.692068) (end 127.076977 67.704784) (width 0.25) (layer "F.Cu") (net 10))
 (segment (start 126.431977 69.054064) (end 129.927913 72.55) (width 0.25) (layer "F.Cu") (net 10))
 (segment (start 127.076977 67.704784) (end 126.431977 68.349784) (width 0.25) (layer "F.Cu") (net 10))
 (segment (start 129.927913 72.55) (end 133.7 72.55) (width 0.25) (layer "F.Cu") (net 10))
 (segment (start 126.431977 68.349784) (end 126.431977 69.054064) (width 0.25) (layer "F.Cu") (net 10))
 (segment (start 127.064261 66.18284) (end 127.064261 67.692068) (width 0.25) (layer "F.Cu") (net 10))
 (segment (start 122.289256 64.883698) (end 122.289256 68.710744) (width 0.25) (layer "F.Cu") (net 2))
 (segment (start 124.839198 63.457839) (end 123.715115 63.457839) (width 0.25) (layer "F.Cu") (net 2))
 (segment (start 122.289256 68.710744) (end 121 70) (width 0.25) (layer "F.Cu") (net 2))
 (segment (start 123.715115 63.457839) (end 122.289256 64.883698) (width 0.25) (layer "F.Cu") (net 2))
 (segment (start 122.739256 70.800744) (end 121 72.54) (width 0.25) (layer "F.Cu") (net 3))
 (segment (start 124.839198 63.95784) (end 123.85151 63.95784) (width 0.25) (layer "F.Cu") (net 3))
 (segment (start 123.85151 63.95784) (end 122.739256 65.070094) (width 0.25) (layer "F.Cu") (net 3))
 (segment (start 122.739256 65.070094) (end 122.739256 70.800744) (width 0.25) (layer "F.Cu") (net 3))
 (segment (start 123.189256 72.890744) (end 121 75.08) (width 0.25) (layer "F.Cu") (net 4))
 (segment (start 123.987906 64.45784) (end 123.189256 65.25649) (width 0.25) (layer "F.Cu") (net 4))
 (segment (start 123.189256 65.25649) (end 123.189256 72.890744) (width 0.25) (layer "F.Cu") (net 4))
 (segment (start 124.839198 64.45784) (end 123.987906 64.45784) (width 0.25) (layer "F.Cu") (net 4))
 (segment (start 124.839198 64.957841) (end 124.124301 64.957841) (width 0.25) (layer "F.Cu") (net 5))
 (segment (start 123.639256 74.980744) (end 121 77.62) (width 0.25) (layer "F.Cu") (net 5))
 (segment (start 124.124301 64.957841) (end 123.639256 65.442886) (width 0.25) (layer "F.Cu") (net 5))
 (segment (start 123.639256 65.442886) (end 123.639256 74.980744) (width 0.25) (layer "F.Cu") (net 5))
 (segment (start 124.839198 65.45784) (end 124.089256 66.207782) (width 0.25) (layer "F.Cu") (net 6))
 (segment (start 124.089256 77.070744) (end 121 80.16) (width 0.25) (layer "F.Cu") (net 6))
 (segment (start 124.089256 66.207782) (end 124.089256 77.070744) (width 0.25) (layer "F.Cu") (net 6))
 (segment (start 125.081977 71.551977) (end 133.7 80.17) (width 0.25) (layer "F.Cu") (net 7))
 (segment (start 125.081977 66.664746) (end 125.081977 71.551977) (width 0.25) (layer "F.Cu") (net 7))
 (segment (start 125.563883 66.18284) (end 125.081977 66.664746) (width 0.25) (layer "F.Cu") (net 7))
 (segment (start 126.064009 67.107076) (end 125.531977 67.639108) (width 0.25) (layer "F.Cu") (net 8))
 (segment (start 125.531977 67.639108) (end 125.531977 69.461977) (width 0.25) (layer "F.Cu") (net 8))
 (segment (start 126.064009 66.18284) (end 126.064009 67.107076) (width 0.25) (layer "F.Cu") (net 8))
 (segment (start 125.531977 69.461977) (end 133.7 77.63) (width 0.25) (layer "F.Cu") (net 8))
 (segment (start 126.564135 67.243346) (end 125.981977 67.825504) (width 0.25) (layer "F.Cu") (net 9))
 (segment (start 125.981977 69.24046) (end 131.831517 75.09) (width 0.25) (layer "F.Cu") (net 9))
 (segment (start 131.831517 75.09) (end 133.7 75.09) (width 0.25) (layer "F.Cu") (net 9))
 (segment (start 125.981977 67.825504) (end 125.981977 69.24046) (width 0.25) (layer "F.Cu") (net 9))
 (segment (start 126.564135 66.18284) (end 126.564135 67.243346) (width 0.25) (layer "F.Cu") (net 9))
 (segment (start 130.356473 70.01) (end 133.7 70.01) (width 0.25) (layer "F.Cu") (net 11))
 (segment (start 127.564387 67.217914) (end 130.356473 70.01) (width 0.25) (layer "F.Cu") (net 11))
 (segment (start 127.564387 66.18284) (end 127.564387 67.217914) (width 0.25) (layer "F.Cu") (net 11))
 (segment (start 128.064513 66.94751) (end 129.117003 68) (width 0.25) (layer "F.Cu") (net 12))
 (segment (start 129.117003 68) (end 133.17 68) (width 0.25) (layer "F.Cu") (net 12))
 (segment (start 128.064513 66.18284) (end 128.064513 66.94751) (width 0.25) (layer "F.Cu") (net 12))
 (segment (start 133.17 68) (end 133.7 67.47) (width 0.25) (layer "F.Cu") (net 12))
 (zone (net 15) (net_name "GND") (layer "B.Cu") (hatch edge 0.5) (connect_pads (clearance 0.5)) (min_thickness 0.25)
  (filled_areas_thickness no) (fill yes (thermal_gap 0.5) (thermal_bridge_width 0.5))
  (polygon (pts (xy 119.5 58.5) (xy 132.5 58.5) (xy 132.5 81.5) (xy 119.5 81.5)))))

